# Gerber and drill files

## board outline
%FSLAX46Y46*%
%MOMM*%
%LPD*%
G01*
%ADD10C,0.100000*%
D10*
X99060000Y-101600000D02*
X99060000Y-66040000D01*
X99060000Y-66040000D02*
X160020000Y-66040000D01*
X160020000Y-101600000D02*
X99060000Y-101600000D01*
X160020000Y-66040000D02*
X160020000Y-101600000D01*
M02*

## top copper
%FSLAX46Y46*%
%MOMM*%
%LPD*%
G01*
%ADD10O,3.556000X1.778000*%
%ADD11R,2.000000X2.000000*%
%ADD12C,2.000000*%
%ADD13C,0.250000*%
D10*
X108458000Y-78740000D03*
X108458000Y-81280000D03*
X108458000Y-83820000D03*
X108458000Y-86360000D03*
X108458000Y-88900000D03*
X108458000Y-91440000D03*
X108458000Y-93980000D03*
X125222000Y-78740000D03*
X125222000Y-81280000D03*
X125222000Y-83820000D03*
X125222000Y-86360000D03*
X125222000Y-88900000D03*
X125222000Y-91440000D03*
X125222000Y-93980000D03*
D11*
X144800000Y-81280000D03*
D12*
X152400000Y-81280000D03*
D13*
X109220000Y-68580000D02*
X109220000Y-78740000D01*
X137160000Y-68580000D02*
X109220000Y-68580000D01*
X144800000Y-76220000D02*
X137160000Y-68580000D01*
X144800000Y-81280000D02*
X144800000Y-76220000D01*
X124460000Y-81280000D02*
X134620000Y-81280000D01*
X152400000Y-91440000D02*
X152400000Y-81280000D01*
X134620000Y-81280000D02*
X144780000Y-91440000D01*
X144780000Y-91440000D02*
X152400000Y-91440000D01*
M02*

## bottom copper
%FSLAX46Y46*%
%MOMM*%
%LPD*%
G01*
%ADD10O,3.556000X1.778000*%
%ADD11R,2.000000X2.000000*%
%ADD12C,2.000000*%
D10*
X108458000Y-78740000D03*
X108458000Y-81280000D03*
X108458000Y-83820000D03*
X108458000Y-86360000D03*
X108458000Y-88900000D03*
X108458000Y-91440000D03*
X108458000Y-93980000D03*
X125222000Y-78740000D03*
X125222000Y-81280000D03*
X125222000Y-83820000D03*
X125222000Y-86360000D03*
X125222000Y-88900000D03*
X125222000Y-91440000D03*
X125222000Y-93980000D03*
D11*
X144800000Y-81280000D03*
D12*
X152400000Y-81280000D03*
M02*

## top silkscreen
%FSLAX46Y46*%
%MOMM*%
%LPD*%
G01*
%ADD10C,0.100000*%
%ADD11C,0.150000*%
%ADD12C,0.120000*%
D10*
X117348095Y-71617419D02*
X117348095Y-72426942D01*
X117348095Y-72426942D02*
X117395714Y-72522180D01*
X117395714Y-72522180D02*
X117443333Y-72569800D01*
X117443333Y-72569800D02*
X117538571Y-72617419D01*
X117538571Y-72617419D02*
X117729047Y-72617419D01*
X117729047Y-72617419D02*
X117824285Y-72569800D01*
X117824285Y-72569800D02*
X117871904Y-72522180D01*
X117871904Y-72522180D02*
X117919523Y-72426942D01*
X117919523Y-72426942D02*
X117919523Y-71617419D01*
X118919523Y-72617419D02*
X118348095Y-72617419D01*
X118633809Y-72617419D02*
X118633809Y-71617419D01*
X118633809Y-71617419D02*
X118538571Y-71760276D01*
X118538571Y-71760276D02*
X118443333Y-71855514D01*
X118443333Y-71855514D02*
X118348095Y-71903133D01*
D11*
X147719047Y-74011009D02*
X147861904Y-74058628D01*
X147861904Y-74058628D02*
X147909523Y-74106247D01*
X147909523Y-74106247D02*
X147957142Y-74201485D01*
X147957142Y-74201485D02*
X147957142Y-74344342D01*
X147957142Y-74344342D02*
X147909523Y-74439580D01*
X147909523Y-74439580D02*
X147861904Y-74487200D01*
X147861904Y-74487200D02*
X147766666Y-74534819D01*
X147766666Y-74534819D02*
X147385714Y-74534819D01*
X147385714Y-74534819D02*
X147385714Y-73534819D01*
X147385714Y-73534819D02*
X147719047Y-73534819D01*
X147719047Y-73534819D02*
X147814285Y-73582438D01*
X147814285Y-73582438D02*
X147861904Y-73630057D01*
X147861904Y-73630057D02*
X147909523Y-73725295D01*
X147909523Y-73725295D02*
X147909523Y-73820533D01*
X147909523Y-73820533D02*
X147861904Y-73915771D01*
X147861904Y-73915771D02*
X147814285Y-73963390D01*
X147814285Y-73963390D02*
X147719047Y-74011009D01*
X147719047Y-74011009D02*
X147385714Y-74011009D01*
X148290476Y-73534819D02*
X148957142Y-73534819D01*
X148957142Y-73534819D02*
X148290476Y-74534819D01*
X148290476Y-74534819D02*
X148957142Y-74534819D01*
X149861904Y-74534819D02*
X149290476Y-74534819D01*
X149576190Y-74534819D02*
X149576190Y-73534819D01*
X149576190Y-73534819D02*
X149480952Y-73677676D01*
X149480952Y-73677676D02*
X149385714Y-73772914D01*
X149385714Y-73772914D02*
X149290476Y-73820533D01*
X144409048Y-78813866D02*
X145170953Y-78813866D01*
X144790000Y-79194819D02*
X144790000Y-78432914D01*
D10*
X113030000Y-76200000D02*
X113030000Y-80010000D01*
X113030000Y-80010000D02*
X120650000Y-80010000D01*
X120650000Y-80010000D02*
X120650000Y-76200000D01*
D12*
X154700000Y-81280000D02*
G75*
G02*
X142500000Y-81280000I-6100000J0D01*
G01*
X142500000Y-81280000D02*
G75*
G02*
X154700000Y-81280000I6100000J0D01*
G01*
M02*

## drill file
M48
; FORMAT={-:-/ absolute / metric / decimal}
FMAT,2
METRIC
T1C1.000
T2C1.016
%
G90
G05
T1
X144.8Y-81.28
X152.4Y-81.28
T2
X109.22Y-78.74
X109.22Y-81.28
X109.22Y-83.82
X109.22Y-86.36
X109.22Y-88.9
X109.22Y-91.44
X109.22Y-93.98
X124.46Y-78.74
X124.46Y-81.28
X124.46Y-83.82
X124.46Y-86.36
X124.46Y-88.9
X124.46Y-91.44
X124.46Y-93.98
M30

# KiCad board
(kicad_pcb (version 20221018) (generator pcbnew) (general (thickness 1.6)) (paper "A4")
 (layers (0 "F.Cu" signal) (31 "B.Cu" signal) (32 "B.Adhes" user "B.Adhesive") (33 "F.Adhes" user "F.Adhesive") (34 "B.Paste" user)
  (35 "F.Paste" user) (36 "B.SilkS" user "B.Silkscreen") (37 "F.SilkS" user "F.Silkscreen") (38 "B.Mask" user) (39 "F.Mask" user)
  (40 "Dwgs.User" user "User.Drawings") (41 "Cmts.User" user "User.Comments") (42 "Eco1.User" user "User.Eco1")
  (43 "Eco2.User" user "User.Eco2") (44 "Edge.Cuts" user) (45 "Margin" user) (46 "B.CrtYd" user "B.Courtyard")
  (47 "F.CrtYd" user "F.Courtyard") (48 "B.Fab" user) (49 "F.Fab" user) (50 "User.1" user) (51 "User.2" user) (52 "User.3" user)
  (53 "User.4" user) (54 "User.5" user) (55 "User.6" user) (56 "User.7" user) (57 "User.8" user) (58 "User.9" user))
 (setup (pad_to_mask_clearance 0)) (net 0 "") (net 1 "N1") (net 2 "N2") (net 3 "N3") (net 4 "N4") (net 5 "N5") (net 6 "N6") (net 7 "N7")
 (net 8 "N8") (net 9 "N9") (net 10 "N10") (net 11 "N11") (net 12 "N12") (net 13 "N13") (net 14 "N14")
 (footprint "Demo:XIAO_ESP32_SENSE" (layer "F.Cu") (at 116.84 86.36)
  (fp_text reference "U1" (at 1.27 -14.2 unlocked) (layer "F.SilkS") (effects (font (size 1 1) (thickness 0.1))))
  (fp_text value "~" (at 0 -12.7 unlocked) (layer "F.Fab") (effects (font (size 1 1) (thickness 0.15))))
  (fp_line (start -3.81 -10.16) (end -3.81 -6.35) (stroke (width 0.1) (type default)) (layer "F.SilkS"))
  (fp_line (start -3.81 -6.35) (end 3.81 -6.35) (stroke (width 0.1) (type default)) (layer "F.SilkS"))
  (fp_line (start 3.81 -6.35) (end 3.81 -10.16) (stroke (width 0.1) (type default)) (layer "F.SilkS"))
  (pad "1" thru_hole oval (at -7.62 -7.62) (size 3.556 1.778) (drill 1.016 (offset -0.762 0)) (layers "*.Cu" "*.Mask") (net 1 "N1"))
  (pad "2" thru_hole oval (at -7.62 -5.08) (size 3.556 1.778) (drill 1.016 (offset -0.762 0)) (layers "*.Cu" "*.Mask") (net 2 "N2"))
  (pad "3" thru_hole oval (at -7.62 -2.54) (size 3.556 1.778) (drill 1.016 (offset -0.762 0)) (layers "*.Cu" "*.Mask") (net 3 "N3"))
  (pad "4" thru_hole oval (at -7.62 0) (size 3.556 1.778) (drill 1.016 (offset -0.762 0)) (layers "*.Cu" "*.Mask") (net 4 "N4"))
  (pad "5" thru_hole oval (at -7.62 2.54) (size 3.556 1.778) (drill 1.016 (offset -0.762 0)) (layers "*.Cu" "*.Mask") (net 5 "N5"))
  (pad "6" thru_hole oval (at -7.62 5.08) (size 3.556 1.778) (drill 1.016 (offset -0.762 0)) (layers "*.Cu" "*.Mask") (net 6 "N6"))
  (pad "7" thru_hole oval (at -7.62 7.62) (size 3.556 1.778) (drill 1.016 (offset -0.762 0)) (layers "*.Cu" "*.Mask") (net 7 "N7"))
  (pad "8" thru_hole oval (at 7.62 -7.62) (size 3.556 1.778) (drill 1.016 (offset 0.762 0)) (layers "*.Cu" "*.Mask") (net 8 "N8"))
  (pad "9" thru_hole oval (at 7.62 -5.08) (size 3.556 1.778) (drill 1.016 (offset 0.762 0)) (layers "*.Cu" "*.Mask") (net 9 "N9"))
  (pad "10" thru_hole oval (at 7.62 -2.54) (size 3.556 1.778) (drill 1.016 (offset 0.762 0)) (layers "*.Cu" "*.Mask") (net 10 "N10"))
  (pad "11" thru_hole oval (at 7.62 0) (size 3.556 1.778) (drill 1.016 (offset 0.762 0)) (layers "*.Cu" "*.Mask") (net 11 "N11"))
  (pad "12" thru_hole oval (at 7.62 2.54) (size 3.556 1.778) (drill 1.016 (offset 0.762 0)) (layers "*.Cu" "*.Mask") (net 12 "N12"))
  (pad "13" thru_hole oval (at 7.62 5.08) (size 3.556 1.778) (drill 1.016 (offset 0.762 0)) (layers "*.Cu" "*.Mask") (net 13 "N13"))
  (pad "14" thru_hole oval (at 7.62 7.62) (size 3.556 1.778) (drill 1.016 (offset 0.762 0)) (layers "*.Cu" "*.Mask") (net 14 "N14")))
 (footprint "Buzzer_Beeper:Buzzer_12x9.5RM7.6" (layer "F.Cu") (at 144.8 81.28)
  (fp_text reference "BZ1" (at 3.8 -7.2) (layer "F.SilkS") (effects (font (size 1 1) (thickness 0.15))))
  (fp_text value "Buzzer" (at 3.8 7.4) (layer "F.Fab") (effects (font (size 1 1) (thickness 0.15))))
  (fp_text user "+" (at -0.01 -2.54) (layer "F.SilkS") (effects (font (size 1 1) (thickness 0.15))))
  (fp_circle (center 3.8 0) (end 9.9 0) (stroke (width 0.12) (type solid)) (fill none) (layer "F.SilkS"))
  (pad "1" thru_hole rect (at 0 0) (size 2 2) (drill 1) (layers "*.Cu" "*.Mask") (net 1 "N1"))
  (pad "2" thru_hole circle (at 7.6 0) (size 2 2) (drill 1) (layers "*.Cu" "*.Mask") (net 9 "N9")))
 (gr_line (start 99.06 101.6) (end 99.06 66.04) (stroke (width 0.1) (type default)) (layer "Edge.Cuts"))
 (gr_line (start 99.06 66.04) (end 160.02 66.04) (stroke (width 0.1) (type default)) (layer "Edge.Cuts"))
 (gr_line (start 160.02 101.6) (end 99.06 101.6) (stroke (width 0.1) (type default)) (layer "Edge.Cuts"))
 (gr_line (start 160.02 66.04) (end 160.02 101.6) (stroke (width 0.1) (type default)) (layer "Edge.Cuts"))
 (segment (start 109.22 68.58) (end 109.22 78.74) (width 0.25) (layer "F.Cu") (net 1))
 (segment (start 137.16 68.58) (end 109.22 68.58) (width 0.25) (layer "F.Cu") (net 1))
 (segment (start 144.8 76.22) (end 137.16 68.58) (width 0.25) (layer "F.Cu") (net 1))
 (segment (start 144.8 81.28) (end 144.8 76.22) (width 0.25) (layer "F.Cu") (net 1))
 (segment (start 124.46 81.28) (end 134.62 81.28) (width 0.25) (layer "F.Cu") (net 9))
 (segment (start 152.4 91.44) (end 152.4 81.28) (width 0.25) (layer "F.Cu") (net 9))
 (segment (start 134.62 81.28) (end 144.78 91.44) (width 0.25) (layer "F.Cu") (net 9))
 (segment (start 144.78 91.44) (end 152.4 91.44) (width 0.25) (layer "F.Cu") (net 9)))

